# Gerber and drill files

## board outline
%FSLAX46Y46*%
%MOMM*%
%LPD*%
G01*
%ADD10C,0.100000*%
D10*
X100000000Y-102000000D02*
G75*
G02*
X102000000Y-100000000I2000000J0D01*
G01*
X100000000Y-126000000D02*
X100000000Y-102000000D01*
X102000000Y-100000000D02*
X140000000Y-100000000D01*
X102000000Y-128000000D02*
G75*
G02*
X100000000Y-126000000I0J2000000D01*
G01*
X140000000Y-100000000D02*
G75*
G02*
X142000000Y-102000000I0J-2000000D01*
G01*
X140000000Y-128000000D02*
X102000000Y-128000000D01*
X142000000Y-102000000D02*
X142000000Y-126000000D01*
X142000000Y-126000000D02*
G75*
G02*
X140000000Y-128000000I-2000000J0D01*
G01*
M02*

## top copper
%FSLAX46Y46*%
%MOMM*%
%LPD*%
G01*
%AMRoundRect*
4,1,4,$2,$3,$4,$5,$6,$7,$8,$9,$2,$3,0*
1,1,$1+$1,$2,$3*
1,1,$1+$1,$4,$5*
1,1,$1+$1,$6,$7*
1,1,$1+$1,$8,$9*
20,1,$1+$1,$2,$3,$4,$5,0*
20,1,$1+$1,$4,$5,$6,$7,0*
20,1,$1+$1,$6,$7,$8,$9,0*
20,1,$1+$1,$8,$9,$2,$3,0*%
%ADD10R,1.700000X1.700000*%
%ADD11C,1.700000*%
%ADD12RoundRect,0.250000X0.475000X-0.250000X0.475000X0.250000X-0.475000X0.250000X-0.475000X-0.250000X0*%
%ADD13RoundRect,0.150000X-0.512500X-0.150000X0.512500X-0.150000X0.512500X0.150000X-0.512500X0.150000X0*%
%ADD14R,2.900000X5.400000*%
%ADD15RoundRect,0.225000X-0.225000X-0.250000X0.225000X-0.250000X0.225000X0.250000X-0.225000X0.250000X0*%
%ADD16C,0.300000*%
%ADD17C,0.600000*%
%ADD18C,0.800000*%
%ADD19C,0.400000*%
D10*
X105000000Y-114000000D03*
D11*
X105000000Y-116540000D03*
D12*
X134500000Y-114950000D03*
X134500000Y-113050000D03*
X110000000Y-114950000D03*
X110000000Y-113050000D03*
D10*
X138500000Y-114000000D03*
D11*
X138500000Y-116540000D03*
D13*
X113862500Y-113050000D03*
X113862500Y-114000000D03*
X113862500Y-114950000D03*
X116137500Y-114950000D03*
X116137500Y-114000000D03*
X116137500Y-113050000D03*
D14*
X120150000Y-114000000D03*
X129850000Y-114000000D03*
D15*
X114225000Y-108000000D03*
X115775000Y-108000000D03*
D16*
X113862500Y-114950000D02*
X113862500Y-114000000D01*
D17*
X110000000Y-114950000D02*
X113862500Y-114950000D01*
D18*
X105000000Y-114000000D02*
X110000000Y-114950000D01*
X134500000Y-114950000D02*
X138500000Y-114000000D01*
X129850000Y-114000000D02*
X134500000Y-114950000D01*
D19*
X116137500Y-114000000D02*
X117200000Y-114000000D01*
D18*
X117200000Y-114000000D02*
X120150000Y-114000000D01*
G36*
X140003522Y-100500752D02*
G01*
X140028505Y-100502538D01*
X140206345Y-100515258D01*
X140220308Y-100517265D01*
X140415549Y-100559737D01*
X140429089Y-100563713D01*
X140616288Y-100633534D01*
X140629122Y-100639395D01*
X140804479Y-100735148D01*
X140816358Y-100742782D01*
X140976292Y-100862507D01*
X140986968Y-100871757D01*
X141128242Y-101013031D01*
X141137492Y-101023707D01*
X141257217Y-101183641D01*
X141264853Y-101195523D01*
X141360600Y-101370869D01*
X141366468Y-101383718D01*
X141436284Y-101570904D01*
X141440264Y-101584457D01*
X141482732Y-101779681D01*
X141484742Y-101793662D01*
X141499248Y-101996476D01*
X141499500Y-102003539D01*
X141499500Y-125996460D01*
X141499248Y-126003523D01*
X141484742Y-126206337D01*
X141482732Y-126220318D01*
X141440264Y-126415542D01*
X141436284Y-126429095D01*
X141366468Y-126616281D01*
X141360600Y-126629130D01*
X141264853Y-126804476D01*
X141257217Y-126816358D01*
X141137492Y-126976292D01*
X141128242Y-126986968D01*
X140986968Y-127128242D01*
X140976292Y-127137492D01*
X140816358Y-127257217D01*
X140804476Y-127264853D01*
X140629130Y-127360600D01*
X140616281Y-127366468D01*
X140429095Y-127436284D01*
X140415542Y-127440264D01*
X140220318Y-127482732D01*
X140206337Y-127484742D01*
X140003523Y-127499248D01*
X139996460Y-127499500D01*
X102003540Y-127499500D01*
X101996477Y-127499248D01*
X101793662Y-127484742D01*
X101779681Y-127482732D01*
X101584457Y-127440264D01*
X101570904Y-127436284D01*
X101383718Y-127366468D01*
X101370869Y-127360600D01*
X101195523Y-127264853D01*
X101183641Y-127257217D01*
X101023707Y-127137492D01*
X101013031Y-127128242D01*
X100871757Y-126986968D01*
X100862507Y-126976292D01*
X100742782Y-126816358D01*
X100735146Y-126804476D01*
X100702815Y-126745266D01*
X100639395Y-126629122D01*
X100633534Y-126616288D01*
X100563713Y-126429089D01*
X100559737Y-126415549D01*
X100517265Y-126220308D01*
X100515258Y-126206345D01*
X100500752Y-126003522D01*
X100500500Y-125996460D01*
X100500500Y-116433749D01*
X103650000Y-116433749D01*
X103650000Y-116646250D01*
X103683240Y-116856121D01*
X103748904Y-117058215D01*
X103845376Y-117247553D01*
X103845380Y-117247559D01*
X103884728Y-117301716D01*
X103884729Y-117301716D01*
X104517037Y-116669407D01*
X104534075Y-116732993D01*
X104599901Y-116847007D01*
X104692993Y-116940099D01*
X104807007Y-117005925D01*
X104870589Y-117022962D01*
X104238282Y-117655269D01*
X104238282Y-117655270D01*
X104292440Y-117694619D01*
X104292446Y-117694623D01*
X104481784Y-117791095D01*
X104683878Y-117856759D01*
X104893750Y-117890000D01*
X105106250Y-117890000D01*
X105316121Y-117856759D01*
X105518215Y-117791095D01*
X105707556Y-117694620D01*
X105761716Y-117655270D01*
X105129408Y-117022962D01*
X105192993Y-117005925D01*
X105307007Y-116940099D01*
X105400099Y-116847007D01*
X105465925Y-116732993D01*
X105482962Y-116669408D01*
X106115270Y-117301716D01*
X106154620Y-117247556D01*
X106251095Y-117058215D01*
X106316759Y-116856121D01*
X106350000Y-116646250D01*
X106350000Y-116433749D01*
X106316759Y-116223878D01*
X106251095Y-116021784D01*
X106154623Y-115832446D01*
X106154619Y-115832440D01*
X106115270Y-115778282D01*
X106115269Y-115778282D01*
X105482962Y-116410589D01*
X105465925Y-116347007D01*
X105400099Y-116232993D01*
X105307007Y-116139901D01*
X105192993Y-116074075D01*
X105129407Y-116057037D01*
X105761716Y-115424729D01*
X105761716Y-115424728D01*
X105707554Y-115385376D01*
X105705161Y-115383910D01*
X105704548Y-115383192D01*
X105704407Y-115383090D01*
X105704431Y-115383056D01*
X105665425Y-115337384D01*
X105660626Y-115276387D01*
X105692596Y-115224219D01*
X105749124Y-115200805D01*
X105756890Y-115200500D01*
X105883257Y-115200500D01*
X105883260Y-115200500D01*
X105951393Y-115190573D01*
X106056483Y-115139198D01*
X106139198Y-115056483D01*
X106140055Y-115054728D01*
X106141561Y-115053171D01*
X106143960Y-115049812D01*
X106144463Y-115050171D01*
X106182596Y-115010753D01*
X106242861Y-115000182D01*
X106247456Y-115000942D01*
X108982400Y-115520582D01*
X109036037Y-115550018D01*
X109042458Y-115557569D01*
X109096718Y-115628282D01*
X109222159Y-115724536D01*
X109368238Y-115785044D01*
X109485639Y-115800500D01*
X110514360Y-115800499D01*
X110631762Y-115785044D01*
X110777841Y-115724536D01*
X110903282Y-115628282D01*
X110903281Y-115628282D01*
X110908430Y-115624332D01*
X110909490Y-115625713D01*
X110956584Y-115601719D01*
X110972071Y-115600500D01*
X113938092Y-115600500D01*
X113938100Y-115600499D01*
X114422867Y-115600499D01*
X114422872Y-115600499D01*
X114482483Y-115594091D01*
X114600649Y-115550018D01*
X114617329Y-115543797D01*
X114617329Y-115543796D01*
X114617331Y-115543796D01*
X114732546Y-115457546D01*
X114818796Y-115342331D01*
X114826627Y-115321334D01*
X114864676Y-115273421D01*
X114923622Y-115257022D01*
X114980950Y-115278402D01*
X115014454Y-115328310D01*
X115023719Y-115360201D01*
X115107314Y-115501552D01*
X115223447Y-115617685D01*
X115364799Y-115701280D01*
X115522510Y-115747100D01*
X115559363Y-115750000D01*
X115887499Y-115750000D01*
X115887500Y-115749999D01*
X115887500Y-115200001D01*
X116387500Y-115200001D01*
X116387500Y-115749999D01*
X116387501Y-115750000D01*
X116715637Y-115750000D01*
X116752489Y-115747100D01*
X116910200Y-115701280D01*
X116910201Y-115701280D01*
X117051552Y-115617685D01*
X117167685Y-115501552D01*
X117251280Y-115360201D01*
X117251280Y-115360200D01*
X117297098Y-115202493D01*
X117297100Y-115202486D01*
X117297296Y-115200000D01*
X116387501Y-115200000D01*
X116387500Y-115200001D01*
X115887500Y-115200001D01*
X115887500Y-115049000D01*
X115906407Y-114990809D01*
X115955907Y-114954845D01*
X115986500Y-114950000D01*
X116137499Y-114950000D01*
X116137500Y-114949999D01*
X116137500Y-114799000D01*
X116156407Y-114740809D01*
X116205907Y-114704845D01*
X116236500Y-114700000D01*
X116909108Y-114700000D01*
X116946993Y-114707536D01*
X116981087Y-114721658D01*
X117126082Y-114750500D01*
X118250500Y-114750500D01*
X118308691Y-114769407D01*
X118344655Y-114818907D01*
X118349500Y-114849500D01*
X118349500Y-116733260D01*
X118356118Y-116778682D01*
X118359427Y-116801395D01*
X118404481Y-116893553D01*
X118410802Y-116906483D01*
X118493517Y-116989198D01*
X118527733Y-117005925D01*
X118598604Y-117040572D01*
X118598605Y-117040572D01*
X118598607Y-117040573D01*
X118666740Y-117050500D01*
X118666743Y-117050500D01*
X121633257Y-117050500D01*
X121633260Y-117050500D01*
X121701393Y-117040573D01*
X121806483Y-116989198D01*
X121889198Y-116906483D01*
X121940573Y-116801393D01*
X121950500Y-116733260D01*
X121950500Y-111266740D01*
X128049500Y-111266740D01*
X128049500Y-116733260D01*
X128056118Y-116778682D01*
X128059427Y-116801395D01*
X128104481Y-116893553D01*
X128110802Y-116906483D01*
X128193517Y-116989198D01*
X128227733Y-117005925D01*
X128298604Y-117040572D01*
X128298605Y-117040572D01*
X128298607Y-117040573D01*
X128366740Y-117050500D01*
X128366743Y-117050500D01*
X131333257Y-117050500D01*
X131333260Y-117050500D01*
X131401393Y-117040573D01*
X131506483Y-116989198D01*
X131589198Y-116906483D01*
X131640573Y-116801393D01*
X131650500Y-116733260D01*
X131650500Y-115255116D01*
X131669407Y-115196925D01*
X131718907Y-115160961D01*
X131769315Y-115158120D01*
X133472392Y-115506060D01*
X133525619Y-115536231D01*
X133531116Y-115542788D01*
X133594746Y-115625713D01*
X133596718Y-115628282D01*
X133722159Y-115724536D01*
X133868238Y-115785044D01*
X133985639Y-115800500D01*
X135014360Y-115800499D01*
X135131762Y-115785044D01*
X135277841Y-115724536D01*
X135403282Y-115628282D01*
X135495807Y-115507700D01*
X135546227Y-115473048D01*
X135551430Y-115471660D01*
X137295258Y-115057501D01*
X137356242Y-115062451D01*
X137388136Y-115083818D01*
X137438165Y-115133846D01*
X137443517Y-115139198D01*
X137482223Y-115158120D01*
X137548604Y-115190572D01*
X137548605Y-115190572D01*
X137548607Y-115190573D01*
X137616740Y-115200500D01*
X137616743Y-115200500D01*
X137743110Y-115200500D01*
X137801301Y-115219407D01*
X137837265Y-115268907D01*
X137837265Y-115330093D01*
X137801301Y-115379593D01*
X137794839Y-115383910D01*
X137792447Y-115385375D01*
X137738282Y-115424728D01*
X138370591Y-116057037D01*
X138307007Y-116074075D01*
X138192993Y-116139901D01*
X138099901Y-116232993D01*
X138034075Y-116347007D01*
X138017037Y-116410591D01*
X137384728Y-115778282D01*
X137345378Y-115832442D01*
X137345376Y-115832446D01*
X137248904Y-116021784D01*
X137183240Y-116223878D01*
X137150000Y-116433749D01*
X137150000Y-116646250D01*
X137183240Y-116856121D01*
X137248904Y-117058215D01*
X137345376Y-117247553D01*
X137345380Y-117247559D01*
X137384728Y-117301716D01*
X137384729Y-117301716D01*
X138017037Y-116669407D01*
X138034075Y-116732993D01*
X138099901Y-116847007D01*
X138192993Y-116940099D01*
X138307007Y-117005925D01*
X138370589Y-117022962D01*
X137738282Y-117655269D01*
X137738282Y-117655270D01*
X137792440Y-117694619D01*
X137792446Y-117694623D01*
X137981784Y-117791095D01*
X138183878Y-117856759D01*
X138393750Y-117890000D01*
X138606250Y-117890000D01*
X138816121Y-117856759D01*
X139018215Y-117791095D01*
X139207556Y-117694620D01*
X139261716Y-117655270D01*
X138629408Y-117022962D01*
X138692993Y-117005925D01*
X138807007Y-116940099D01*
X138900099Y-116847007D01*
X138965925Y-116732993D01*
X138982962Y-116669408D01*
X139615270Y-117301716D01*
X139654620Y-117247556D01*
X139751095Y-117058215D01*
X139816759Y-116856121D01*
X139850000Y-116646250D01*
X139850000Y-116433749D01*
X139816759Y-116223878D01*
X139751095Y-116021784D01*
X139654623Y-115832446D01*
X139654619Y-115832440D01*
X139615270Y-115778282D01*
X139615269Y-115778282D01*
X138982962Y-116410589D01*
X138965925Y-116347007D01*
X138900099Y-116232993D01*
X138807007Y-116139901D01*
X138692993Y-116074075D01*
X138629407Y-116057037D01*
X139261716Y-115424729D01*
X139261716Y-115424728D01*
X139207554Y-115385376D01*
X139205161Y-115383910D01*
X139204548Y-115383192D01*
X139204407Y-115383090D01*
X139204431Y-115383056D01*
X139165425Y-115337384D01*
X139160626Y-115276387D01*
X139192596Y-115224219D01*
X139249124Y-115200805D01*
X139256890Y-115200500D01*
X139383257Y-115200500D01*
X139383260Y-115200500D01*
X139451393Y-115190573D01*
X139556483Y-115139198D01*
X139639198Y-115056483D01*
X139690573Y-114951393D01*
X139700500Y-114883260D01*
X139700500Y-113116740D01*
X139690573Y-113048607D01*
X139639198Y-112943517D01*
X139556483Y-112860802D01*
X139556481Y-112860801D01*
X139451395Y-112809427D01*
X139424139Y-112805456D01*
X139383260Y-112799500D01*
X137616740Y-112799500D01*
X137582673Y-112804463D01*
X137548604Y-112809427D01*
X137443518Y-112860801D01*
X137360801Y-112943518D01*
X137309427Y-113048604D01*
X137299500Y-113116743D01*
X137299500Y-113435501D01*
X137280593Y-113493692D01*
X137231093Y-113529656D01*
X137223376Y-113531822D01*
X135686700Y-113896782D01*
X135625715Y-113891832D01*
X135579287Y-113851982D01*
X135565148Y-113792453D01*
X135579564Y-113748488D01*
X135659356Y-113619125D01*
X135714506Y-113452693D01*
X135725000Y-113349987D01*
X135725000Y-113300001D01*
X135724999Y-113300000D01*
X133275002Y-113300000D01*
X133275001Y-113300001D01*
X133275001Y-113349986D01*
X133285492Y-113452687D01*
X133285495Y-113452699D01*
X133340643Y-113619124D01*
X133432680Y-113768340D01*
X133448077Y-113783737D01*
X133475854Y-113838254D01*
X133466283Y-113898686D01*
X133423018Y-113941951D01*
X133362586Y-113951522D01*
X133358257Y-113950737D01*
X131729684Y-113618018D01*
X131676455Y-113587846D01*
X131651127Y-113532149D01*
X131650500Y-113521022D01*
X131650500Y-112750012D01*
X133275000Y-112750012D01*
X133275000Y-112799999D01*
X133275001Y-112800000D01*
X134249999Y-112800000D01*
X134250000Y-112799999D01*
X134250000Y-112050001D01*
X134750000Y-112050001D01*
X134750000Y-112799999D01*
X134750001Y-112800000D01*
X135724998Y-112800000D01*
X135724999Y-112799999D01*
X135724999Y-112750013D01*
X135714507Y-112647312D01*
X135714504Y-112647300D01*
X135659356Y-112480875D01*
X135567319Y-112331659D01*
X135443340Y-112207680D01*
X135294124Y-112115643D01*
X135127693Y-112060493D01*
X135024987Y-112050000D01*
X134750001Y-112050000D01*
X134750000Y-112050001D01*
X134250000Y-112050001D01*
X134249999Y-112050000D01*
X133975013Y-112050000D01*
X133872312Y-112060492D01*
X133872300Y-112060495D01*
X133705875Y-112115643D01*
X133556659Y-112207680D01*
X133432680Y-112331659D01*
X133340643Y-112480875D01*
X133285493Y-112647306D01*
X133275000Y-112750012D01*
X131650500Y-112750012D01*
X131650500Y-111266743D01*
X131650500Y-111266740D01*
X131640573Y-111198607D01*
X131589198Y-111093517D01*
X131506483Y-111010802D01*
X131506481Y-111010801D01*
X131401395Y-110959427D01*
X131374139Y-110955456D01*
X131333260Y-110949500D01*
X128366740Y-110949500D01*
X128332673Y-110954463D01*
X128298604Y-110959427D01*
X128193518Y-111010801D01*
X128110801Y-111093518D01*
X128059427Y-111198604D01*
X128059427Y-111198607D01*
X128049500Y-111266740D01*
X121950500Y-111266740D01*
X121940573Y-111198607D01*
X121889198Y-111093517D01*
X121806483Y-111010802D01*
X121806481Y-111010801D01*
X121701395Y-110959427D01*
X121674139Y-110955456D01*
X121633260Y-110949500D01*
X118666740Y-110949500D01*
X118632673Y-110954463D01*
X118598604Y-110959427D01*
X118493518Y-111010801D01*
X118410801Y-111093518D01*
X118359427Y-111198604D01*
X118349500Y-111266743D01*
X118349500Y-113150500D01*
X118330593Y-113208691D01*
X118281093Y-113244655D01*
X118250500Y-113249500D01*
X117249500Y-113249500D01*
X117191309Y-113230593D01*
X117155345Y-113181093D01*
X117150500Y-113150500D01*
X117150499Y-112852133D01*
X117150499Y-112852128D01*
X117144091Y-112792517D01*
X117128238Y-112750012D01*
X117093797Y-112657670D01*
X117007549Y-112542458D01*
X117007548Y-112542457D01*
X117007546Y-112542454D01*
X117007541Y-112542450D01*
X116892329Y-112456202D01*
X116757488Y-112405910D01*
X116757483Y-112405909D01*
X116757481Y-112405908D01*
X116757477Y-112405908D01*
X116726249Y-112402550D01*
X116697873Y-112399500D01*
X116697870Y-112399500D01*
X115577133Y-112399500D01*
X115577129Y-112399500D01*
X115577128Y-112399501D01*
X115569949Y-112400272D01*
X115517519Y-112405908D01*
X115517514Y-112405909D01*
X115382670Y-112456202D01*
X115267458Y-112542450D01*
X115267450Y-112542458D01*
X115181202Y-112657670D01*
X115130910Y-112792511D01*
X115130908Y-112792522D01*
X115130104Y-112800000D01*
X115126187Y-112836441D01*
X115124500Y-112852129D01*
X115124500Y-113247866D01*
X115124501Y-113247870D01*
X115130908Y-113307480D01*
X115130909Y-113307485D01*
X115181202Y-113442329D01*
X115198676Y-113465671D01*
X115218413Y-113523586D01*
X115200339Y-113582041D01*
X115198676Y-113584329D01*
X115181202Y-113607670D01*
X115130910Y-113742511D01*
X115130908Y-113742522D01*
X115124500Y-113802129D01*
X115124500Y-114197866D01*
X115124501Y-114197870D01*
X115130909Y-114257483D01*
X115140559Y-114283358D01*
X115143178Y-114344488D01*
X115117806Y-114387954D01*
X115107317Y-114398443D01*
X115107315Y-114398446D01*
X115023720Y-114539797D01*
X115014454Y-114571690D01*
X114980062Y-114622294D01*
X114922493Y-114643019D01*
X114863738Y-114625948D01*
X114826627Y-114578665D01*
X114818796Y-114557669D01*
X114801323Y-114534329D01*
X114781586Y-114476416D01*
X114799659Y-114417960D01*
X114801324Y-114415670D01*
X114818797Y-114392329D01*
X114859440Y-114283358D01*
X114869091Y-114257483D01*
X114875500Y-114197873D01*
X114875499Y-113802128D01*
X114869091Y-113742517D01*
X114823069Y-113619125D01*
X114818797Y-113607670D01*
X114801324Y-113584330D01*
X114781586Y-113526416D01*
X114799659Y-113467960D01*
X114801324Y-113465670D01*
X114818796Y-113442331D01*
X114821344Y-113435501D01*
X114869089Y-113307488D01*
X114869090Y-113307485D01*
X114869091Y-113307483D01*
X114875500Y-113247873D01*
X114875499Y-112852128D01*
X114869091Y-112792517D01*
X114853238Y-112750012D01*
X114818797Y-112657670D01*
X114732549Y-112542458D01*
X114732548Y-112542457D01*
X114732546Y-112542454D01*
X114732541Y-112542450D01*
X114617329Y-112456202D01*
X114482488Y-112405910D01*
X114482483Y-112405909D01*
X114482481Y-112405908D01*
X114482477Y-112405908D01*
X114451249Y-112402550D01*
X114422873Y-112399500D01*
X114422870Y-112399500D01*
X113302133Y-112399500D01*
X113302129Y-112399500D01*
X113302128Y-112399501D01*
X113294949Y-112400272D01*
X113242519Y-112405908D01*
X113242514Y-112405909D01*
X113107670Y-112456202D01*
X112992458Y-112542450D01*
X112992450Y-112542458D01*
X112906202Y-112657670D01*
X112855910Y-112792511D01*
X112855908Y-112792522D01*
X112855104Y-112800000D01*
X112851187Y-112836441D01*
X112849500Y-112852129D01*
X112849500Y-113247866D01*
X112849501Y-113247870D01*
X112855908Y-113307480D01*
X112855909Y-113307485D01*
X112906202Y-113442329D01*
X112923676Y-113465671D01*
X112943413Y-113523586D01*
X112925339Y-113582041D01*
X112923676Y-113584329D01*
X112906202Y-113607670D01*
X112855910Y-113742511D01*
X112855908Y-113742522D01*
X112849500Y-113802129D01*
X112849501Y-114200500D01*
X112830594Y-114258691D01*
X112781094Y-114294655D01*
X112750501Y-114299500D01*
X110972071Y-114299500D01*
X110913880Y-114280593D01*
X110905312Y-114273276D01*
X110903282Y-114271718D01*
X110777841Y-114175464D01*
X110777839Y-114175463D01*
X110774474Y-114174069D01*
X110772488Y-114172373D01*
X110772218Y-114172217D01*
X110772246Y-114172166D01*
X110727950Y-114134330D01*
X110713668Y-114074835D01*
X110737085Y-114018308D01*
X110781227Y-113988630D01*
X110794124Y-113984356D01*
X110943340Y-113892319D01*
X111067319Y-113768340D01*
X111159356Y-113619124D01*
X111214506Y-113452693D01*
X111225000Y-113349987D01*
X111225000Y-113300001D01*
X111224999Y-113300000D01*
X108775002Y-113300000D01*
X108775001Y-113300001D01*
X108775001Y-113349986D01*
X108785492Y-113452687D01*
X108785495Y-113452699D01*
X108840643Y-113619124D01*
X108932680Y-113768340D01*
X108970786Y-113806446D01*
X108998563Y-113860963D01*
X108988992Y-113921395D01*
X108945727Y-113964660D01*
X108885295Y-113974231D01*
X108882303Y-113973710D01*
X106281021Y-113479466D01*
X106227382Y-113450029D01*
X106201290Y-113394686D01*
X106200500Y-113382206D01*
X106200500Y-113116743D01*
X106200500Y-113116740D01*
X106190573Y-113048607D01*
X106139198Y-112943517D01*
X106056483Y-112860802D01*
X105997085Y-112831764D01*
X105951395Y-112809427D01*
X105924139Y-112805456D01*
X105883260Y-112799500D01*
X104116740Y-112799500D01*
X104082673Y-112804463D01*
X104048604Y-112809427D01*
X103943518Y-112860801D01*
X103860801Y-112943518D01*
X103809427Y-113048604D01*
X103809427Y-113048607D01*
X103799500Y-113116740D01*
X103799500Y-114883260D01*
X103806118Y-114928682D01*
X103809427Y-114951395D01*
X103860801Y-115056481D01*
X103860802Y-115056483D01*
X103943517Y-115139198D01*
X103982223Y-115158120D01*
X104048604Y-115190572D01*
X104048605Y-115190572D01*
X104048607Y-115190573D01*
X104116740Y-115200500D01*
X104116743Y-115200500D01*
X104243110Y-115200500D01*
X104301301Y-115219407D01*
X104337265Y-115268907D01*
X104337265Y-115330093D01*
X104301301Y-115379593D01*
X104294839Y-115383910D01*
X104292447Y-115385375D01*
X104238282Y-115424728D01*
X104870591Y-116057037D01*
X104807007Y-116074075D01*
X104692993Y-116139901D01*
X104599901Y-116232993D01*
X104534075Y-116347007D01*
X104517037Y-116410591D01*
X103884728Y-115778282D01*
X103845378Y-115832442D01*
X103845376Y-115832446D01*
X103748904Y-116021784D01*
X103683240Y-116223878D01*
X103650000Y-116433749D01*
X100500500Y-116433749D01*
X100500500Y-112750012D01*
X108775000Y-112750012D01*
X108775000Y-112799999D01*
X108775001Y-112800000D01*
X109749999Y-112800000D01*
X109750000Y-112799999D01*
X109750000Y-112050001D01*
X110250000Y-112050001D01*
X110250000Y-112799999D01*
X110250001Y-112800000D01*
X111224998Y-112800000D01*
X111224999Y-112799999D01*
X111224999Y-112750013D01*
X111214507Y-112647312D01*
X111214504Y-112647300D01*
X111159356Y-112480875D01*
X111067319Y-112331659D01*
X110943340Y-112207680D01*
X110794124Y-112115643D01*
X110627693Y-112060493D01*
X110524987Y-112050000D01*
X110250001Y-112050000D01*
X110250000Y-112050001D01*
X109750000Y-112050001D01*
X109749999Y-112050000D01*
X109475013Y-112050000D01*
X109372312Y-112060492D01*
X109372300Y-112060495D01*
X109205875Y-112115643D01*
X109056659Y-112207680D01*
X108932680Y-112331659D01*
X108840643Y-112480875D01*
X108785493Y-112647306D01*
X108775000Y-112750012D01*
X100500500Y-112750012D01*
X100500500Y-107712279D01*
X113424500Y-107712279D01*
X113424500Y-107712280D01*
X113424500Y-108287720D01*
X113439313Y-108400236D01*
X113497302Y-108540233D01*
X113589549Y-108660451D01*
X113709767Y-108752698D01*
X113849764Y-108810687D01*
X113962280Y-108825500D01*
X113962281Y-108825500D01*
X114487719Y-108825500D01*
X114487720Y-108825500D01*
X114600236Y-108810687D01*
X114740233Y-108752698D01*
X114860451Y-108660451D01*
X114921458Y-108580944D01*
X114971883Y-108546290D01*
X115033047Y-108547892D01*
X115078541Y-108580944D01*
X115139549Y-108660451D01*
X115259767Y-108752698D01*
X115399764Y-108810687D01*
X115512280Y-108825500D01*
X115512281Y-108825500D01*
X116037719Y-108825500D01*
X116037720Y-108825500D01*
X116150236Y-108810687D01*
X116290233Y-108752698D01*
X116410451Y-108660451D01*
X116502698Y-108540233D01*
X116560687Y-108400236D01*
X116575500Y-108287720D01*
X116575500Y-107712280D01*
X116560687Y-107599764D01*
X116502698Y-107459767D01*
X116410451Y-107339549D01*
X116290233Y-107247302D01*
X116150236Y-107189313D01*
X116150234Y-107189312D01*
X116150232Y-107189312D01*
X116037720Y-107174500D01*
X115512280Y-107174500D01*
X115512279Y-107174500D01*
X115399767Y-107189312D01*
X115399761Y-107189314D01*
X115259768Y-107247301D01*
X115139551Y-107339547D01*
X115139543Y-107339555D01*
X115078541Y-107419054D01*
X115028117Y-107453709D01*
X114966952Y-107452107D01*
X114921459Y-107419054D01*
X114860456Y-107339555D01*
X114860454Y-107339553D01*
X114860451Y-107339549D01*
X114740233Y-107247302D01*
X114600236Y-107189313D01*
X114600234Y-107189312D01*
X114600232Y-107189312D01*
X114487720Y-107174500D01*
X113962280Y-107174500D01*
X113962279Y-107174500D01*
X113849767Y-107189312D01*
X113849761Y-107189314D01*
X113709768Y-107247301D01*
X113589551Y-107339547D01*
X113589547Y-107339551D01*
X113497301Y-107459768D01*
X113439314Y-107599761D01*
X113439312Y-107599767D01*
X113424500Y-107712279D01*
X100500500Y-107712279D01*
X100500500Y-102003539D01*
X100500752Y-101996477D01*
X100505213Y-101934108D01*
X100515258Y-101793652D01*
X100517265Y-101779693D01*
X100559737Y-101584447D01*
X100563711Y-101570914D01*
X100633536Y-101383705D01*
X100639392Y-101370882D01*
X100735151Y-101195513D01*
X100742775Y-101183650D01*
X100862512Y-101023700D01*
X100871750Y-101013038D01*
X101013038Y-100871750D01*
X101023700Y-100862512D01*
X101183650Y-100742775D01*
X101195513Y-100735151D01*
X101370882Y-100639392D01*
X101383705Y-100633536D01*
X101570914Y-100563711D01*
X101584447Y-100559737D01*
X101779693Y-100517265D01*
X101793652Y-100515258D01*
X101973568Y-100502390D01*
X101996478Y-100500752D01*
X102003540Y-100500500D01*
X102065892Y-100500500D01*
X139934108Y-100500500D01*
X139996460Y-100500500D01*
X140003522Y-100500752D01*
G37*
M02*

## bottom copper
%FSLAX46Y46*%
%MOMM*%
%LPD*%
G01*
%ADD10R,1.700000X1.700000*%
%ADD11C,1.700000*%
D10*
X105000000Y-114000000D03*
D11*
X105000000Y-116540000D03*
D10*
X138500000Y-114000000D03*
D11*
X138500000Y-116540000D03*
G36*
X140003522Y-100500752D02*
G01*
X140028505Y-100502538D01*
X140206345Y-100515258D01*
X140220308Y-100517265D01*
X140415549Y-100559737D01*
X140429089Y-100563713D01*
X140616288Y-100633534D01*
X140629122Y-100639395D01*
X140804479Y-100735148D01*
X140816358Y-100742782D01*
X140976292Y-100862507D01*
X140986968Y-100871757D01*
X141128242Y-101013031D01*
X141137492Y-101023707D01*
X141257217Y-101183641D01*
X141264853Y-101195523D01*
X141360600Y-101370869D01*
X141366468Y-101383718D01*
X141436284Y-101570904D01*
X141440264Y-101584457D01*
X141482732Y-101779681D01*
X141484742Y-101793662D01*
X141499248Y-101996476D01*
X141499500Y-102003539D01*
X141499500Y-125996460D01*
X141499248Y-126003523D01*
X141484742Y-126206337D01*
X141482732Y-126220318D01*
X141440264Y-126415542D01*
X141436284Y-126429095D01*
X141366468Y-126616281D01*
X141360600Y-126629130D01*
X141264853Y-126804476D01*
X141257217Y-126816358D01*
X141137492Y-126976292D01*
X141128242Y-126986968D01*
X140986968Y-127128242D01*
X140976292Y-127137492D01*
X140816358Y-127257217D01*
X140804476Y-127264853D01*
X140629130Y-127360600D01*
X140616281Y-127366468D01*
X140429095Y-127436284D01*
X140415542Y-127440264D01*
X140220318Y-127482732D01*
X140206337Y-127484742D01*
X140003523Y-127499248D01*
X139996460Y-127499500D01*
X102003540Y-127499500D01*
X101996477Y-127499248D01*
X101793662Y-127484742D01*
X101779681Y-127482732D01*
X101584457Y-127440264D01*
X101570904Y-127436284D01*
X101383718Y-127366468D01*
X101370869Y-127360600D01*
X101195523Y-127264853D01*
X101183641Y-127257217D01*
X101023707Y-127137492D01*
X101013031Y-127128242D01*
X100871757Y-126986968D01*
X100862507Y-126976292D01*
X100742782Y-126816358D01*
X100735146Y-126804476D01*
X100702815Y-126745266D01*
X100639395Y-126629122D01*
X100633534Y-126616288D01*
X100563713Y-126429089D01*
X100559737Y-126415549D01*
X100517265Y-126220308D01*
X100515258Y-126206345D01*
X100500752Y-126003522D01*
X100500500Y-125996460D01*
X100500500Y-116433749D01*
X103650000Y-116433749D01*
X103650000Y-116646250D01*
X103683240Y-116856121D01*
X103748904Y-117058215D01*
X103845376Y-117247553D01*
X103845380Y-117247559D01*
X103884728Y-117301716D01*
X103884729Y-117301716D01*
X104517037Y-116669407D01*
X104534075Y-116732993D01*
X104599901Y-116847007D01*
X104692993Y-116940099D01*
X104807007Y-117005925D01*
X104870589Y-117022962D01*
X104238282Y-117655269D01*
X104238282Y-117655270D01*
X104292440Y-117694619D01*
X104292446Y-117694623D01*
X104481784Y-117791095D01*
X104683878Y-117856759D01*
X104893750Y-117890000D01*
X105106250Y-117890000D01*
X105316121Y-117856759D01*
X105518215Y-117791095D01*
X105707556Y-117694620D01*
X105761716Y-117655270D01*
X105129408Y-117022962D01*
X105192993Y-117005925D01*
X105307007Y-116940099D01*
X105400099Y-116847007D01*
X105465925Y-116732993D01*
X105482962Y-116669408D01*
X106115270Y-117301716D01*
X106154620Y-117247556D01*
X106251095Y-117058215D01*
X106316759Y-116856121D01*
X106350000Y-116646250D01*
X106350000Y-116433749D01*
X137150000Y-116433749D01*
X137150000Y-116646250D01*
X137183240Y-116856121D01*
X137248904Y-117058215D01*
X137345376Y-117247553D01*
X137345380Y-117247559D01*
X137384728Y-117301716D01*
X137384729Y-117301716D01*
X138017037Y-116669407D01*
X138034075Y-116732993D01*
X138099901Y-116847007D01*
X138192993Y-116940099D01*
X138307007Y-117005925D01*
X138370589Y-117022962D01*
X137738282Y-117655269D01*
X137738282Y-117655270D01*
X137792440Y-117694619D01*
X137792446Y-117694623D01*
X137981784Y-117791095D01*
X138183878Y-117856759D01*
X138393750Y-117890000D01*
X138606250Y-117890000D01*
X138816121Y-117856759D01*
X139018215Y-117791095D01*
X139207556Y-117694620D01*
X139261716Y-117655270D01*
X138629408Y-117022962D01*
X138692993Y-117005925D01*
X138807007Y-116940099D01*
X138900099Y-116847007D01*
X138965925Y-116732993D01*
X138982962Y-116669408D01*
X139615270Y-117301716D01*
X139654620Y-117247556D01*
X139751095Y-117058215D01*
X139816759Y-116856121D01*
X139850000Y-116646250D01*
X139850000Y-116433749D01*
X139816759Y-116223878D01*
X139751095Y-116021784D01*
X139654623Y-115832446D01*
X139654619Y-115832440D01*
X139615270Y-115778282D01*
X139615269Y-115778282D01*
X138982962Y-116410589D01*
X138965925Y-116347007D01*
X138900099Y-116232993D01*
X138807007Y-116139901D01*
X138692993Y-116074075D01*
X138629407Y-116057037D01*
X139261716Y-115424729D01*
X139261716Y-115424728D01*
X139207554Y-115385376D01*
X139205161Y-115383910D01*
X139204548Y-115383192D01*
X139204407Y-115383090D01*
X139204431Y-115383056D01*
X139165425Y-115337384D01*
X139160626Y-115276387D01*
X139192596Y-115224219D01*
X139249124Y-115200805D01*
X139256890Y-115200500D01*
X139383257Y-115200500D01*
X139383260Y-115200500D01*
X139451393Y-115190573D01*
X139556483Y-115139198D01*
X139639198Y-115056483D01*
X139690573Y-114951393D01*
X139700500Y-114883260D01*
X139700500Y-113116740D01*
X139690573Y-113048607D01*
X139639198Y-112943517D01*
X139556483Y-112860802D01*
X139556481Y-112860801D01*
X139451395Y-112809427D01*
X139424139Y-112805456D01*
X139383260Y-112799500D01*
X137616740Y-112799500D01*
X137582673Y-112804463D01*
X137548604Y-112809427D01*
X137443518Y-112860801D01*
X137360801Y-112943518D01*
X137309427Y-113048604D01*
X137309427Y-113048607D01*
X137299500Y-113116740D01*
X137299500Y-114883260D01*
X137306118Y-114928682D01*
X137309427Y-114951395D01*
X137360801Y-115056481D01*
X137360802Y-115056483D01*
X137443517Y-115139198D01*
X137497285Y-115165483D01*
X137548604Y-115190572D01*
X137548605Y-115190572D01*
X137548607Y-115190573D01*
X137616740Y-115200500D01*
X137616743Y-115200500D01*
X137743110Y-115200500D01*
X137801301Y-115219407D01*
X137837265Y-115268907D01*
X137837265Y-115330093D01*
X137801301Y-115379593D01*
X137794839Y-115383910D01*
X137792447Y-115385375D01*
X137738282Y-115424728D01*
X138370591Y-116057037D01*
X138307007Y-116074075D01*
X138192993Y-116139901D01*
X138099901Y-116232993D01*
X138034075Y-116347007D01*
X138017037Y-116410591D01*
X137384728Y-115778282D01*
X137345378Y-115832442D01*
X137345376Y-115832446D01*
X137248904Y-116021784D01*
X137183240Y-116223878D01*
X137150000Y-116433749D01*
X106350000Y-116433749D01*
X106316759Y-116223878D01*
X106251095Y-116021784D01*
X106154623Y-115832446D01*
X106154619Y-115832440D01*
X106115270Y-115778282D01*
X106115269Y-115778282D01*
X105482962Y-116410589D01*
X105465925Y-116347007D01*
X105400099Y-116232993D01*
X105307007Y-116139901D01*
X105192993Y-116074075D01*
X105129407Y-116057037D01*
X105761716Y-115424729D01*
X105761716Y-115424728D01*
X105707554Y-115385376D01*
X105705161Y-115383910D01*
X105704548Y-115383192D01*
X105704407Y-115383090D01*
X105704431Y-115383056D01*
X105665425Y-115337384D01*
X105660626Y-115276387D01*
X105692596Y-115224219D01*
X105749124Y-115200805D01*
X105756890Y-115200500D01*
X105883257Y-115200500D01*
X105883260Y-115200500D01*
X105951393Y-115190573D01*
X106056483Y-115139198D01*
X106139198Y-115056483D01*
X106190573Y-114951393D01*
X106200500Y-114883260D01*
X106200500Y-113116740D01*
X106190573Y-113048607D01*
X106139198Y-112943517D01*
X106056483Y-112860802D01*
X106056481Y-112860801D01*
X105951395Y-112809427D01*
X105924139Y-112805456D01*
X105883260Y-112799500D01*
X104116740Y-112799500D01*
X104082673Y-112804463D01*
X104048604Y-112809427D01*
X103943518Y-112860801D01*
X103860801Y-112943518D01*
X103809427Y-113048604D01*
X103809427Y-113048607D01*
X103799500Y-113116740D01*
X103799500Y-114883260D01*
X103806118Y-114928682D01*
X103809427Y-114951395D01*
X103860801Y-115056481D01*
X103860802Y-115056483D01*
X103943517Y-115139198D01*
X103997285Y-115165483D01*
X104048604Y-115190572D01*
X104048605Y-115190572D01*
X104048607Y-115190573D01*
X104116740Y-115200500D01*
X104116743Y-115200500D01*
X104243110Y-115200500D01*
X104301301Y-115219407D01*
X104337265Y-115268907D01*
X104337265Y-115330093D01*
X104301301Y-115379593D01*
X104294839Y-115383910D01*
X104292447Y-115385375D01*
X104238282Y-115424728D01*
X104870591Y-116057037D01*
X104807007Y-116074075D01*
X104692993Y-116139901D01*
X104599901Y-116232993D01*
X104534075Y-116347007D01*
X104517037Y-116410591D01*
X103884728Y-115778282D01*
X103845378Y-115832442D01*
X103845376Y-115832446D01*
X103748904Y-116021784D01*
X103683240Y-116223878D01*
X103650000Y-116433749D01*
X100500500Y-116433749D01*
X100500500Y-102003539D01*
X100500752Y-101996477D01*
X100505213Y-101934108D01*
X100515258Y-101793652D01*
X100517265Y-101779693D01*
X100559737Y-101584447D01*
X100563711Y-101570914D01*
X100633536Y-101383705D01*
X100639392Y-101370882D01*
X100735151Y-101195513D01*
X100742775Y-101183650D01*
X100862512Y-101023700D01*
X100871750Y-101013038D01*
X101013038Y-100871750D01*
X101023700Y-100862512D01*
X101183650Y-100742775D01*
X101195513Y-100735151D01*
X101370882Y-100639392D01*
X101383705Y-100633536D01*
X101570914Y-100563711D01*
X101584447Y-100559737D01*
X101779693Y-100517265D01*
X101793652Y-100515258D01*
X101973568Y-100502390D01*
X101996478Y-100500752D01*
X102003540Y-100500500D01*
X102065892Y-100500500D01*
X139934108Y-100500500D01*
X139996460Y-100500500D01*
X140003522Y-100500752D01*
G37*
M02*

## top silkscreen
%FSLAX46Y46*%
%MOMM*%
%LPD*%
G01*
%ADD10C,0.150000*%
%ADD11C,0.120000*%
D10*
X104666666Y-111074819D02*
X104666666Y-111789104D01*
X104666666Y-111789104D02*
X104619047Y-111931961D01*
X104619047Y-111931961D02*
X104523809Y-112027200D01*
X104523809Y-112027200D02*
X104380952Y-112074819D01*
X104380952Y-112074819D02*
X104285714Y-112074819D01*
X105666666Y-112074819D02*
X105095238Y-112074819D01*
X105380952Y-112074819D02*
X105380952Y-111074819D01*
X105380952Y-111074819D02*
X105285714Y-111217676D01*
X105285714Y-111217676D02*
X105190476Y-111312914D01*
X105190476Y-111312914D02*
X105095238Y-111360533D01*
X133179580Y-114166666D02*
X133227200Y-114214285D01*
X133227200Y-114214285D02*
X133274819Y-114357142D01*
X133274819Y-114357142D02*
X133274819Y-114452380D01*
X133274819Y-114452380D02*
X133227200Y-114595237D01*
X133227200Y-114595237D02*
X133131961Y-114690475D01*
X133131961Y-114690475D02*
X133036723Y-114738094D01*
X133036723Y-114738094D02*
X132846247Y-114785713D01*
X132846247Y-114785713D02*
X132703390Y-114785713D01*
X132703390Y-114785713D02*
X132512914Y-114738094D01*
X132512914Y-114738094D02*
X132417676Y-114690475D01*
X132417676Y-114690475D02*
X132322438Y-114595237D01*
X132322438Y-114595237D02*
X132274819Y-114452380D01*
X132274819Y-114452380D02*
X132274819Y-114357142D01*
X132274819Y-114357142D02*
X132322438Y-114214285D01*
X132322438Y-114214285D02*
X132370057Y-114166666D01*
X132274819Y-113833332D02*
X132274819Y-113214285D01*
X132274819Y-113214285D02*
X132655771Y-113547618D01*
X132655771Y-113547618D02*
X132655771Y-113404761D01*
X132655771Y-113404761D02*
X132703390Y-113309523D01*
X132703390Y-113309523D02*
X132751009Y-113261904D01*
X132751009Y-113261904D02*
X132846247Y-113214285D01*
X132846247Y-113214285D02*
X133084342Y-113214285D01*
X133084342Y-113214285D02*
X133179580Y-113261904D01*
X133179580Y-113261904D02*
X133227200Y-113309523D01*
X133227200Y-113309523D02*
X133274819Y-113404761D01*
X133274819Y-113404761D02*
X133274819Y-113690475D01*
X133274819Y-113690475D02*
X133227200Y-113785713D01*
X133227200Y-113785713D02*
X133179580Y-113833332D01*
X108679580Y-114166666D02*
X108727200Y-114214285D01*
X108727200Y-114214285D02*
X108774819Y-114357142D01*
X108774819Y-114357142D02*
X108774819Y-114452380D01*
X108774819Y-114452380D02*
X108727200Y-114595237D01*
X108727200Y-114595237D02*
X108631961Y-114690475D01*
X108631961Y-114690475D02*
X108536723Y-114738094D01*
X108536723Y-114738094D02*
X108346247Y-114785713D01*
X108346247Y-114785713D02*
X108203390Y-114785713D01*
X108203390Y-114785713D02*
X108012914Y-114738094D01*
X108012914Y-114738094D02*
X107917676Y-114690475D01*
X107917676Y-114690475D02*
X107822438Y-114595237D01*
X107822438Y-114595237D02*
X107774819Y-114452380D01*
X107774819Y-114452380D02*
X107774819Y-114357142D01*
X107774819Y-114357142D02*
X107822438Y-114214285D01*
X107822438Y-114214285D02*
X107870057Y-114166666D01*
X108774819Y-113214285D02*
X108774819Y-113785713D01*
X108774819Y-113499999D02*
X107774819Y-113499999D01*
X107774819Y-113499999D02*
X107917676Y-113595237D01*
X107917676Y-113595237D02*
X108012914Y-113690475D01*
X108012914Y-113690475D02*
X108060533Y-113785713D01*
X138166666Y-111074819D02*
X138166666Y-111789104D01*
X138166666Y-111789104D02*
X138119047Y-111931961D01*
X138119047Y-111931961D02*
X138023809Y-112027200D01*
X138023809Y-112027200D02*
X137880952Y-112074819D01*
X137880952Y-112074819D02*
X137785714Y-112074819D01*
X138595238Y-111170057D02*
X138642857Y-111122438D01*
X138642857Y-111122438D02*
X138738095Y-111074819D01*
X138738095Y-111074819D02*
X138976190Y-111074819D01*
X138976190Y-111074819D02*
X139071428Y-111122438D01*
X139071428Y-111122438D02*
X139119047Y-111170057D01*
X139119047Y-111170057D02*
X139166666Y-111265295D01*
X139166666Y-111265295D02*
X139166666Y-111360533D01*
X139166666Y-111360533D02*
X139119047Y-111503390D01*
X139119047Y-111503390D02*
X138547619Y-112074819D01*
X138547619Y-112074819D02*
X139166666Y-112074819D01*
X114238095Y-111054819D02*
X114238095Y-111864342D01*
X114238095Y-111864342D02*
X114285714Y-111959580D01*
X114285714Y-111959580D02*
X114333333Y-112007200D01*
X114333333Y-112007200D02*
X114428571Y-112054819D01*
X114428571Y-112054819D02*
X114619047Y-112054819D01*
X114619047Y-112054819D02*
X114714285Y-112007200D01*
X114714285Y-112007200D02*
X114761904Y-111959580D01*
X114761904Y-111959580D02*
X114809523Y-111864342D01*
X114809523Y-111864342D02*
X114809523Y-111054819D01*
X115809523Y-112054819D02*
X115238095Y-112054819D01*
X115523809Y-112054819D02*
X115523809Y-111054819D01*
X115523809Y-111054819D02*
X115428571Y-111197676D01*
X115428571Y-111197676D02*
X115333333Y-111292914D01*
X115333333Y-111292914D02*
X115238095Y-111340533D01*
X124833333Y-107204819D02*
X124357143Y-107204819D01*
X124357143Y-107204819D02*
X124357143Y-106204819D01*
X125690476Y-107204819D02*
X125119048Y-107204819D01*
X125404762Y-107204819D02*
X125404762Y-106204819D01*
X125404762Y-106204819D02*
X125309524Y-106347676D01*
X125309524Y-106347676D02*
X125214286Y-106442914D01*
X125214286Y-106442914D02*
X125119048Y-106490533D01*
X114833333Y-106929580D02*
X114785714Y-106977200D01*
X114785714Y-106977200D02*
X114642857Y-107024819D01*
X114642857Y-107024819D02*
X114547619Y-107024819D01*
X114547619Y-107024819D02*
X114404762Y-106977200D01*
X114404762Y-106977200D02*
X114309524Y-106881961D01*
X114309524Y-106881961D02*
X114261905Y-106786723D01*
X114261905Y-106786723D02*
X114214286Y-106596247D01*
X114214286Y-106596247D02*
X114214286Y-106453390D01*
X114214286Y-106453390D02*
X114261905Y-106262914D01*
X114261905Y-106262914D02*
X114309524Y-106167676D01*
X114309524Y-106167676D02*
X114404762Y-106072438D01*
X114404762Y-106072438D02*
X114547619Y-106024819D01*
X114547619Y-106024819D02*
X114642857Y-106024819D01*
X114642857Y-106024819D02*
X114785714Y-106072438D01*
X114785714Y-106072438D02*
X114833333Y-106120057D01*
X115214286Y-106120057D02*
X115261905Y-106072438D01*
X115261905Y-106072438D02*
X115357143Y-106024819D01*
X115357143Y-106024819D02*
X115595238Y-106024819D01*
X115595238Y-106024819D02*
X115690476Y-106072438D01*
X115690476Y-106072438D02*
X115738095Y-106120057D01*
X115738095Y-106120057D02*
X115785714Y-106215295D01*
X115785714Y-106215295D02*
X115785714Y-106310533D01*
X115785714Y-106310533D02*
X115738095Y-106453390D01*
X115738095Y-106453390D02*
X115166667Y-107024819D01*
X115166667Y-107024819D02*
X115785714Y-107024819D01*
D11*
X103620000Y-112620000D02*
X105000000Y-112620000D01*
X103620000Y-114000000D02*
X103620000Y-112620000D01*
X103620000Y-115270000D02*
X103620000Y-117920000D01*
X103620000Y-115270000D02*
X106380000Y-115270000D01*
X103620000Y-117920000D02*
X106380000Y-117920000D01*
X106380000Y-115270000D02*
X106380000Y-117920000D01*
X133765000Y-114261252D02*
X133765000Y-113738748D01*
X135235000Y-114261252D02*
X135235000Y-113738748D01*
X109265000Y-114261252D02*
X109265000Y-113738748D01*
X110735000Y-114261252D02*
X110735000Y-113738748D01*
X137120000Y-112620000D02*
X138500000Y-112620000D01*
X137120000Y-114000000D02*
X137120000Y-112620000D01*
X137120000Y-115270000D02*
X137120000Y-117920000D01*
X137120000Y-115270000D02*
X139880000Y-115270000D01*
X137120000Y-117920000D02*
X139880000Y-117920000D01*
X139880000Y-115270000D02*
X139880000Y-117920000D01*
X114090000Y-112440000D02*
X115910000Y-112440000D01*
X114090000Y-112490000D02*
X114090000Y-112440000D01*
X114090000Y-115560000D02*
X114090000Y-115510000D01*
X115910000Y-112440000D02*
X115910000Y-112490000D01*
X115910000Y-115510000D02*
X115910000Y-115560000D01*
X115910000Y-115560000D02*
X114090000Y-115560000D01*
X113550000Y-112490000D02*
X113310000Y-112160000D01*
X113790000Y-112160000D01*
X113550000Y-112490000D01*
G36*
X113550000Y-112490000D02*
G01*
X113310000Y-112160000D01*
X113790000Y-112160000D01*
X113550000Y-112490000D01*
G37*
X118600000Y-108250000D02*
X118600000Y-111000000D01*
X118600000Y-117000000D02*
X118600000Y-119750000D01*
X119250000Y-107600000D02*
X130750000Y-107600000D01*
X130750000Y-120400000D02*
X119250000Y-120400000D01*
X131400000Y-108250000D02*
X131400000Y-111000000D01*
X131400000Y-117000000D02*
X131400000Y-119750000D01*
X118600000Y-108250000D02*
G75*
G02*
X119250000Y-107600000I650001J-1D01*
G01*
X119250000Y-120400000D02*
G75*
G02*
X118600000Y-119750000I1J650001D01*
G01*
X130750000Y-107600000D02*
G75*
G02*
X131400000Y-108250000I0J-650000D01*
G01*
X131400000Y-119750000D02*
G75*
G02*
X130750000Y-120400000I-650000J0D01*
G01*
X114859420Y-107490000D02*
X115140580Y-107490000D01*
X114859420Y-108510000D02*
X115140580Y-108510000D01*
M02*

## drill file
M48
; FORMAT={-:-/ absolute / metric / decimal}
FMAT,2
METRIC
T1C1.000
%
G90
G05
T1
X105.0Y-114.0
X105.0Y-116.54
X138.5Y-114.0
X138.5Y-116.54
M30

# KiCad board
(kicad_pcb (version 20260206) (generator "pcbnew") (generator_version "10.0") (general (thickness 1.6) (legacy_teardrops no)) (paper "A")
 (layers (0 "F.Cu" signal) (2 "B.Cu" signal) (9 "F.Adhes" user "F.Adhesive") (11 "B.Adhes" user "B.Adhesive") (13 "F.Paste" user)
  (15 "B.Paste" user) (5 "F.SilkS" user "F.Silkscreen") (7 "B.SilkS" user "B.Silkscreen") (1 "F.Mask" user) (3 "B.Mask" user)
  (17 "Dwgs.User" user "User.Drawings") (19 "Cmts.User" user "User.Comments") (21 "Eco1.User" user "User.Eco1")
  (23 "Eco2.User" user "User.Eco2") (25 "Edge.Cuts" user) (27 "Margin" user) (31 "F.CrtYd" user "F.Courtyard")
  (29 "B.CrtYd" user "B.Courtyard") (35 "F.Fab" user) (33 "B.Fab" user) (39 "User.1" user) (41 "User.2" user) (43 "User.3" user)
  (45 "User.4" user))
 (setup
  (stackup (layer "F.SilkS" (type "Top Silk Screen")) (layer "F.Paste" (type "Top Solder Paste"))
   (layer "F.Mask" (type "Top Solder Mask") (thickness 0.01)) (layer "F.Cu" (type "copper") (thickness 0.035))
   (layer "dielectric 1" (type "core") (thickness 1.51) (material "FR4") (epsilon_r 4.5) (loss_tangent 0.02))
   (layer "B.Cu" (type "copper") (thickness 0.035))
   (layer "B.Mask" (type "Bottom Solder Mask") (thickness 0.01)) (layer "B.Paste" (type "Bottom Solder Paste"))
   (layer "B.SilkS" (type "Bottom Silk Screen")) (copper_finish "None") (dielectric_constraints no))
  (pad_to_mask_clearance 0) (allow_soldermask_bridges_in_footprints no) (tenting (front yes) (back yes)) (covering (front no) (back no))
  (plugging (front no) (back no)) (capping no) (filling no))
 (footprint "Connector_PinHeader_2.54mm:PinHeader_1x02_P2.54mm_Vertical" (layer "F.Cu") (at 105 114)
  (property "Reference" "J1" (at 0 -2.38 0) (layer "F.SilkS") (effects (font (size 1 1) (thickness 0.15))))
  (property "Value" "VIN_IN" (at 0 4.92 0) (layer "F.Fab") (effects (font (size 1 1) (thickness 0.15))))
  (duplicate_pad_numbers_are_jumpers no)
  (fp_line (start -1.38 -1.38) (end 0 -1.38) (stroke (width 0.12) (type solid)) (layer "F.SilkS"))
  (fp_line (start -1.38 0) (end -1.38 -1.38) (stroke (width 0.12) (type solid)) (layer "F.SilkS"))
  (fp_line (start -1.38 1.27) (end -1.38 3.92) (stroke (width 0.12) (type solid)) (layer "F.SilkS"))
  (fp_line (start -1.38 1.27) (end 1.38 1.27) (stroke (width 0.12) (type solid)) (layer "F.SilkS"))
  (fp_line (start -1.38 3.92) (end 1.38 3.92) (stroke (width 0.12) (type solid)) (layer "F.SilkS"))
  (fp_line (start 1.38 1.27) (end 1.38 3.92) (stroke (width 0.12) (type solid)) (layer "F.SilkS"))
  (pad "1" thru_hole rect (at 0 0) (size 1.7 1.7) (drill 1) (layers "*.Cu" "*.Mask") (remove_unused_layers no) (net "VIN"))
  (pad "2" thru_hole circle (at 0 2.54) (size 1.7 1.7) (drill 1) (layers "*.Cu" "*.Mask") (remove_unused_layers no) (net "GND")))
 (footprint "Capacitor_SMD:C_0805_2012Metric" (layer "F.Cu") (at 134.5 114 90)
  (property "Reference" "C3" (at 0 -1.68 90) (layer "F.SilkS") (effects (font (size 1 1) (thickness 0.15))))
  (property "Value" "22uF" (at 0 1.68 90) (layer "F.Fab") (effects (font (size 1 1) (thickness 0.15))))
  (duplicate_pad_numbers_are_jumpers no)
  (fp_line (start -0.261252 -0.735) (end 0.261252 -0.735) (stroke (width 0.12) (type solid)) (layer "F.SilkS"))
  (fp_line (start -0.261252 0.735) (end 0.261252 0.735) (stroke (width 0.12) (type solid)) (layer "F.SilkS"))
  (pad "1" smd roundrect (at -0.95 0 90) (size 1 1.45) (layers "F.Cu" "F.Mask" "F.Paste") (roundrect_rratio 0.25) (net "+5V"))
  (pad "2" smd roundrect (at 0.95 0 90) (size 1 1.45) (layers "F.Cu" "F.Mask" "F.Paste") (roundrect_rratio 0.25) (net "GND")))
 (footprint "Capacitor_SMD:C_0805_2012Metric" (layer "F.Cu") (at 110 114 90)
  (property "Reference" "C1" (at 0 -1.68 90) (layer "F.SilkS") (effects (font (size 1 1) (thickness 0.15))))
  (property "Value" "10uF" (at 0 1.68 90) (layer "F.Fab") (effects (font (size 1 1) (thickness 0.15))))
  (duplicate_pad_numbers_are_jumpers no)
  (fp_line (start -0.261252 -0.735) (end 0.261252 -0.735) (stroke (width 0.12) (type solid)) (layer "F.SilkS"))
  (fp_line (start -0.261252 0.735) (end 0.261252 0.735) (stroke (width 0.12) (type solid)) (layer "F.SilkS"))
  (pad "1" smd roundrect (at -0.95 0 90) (size 1 1.45) (layers "F.Cu" "F.Mask" "F.Paste") (roundrect_rratio 0.25) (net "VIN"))
  (pad "2" smd roundrect (at 0.95 0 90) (size 1 1.45) (layers "F.Cu" "F.Mask" "F.Paste") (roundrect_rratio 0.25) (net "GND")))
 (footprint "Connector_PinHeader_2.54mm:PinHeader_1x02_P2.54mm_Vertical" (layer "F.Cu") (at 138.5 114)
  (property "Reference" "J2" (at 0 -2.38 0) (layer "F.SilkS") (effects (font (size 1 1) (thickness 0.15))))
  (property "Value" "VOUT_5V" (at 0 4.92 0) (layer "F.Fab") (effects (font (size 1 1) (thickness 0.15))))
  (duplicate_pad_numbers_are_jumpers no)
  (fp_line (start -1.38 -1.38) (end 0 -1.38) (stroke (width 0.12) (type solid)) (layer "F.SilkS"))
  (fp_line (start -1.38 0) (end -1.38 -1.38) (stroke (width 0.12) (type solid)) (layer "F.SilkS"))
  (fp_line (start -1.38 1.27) (end -1.38 3.92) (stroke (width 0.12) (type solid)) (layer "F.SilkS"))
  (fp_line (start -1.38 1.27) (end 1.38 1.27) (stroke (width 0.12) (type solid)) (layer "F.SilkS"))
  (fp_line (start -1.38 3.92) (end 1.38 3.92) (stroke (width 0.12) (type solid)) (layer "F.SilkS"))
  (fp_line (start 1.38 1.27) (end 1.38 3.92) (stroke (width 0.12) (type solid)) (layer "F.SilkS"))
  (pad "1" thru_hole rect (at 0 0) (size 1.7 1.7) (drill 1) (layers "*.Cu" "*.Mask") (remove_unused_layers no) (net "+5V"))
  (pad "2" thru_hole circle (at 0 2.54) (size 1.7 1.7) (drill 1) (layers "*.Cu" "*.Mask") (remove_unused_layers no) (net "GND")))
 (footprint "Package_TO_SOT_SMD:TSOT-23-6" (layer "F.Cu") (at 115 114)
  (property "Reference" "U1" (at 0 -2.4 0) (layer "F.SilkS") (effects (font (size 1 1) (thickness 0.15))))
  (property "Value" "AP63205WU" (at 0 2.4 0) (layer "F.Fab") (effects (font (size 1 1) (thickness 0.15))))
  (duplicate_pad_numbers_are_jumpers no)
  (fp_line (start -0.91 -1.56) (end 0.91 -1.56) (stroke (width 0.12) (type solid)) (layer "F.SilkS"))
  (fp_line (start -0.91 -1.51) (end -0.91 -1.56) (stroke (width 0.12) (type solid)) (layer "F.SilkS"))
  (fp_line (start -0.91 1.56) (end -0.91 1.51) (stroke (width 0.12) (type solid)) (layer "F.SilkS"))
  (fp_line (start 0.91 -1.56) (end 0.91 -1.51) (stroke (width 0.12) (type solid)) (layer "F.SilkS"))
  (fp_line (start 0.91 1.51) (end 0.91 1.56) (stroke (width 0.12) (type solid)) (layer "F.SilkS"))
  (fp_line (start 0.91 1.56) (end -0.91 1.56) (stroke (width 0.12) (type solid)) (layer "F.SilkS"))
  (fp_poly (pts (xy -1.45 -1.51) (xy -1.69 -1.84) (xy -1.21 -1.84)) (stroke (width 0.12) (type solid)) (fill yes) (layer "F.SilkS"))
  (pad "1" smd roundrect (at -1.1375 -0.95) (size 1.325 0.6) (layers "F.Cu" "F.Mask" "F.Paste") (roundrect_rratio 0.25) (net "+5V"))
  (pad "2" smd roundrect (at -1.1375 0) (size 1.325 0.6) (layers "F.Cu" "F.Mask" "F.Paste") (roundrect_rratio 0.25) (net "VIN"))
  (pad "3" smd roundrect (at -1.1375 0.95) (size 1.325 0.6) (layers "F.Cu" "F.Mask" "F.Paste") (roundrect_rratio 0.25) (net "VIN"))
  (pad "4" smd roundrect (at 1.1375 0.95) (size 1.325 0.6) (layers "F.Cu" "F.Mask" "F.Paste") (roundrect_rratio 0.25) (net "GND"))
  (pad "5" smd roundrect (at 1.1375 0) (size 1.325 0.6) (layers "F.Cu" "F.Mask" "F.Paste") (roundrect_rratio 0.25) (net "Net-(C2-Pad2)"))
  (pad "6" smd roundrect (at 1.1375 -0.95) (size 1.325 0.6) (layers "F.Cu" "F.Mask" "F.Paste") (roundrect_rratio 0.25) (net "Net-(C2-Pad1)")))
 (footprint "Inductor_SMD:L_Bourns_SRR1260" (layer "F.Cu") (at 125 114)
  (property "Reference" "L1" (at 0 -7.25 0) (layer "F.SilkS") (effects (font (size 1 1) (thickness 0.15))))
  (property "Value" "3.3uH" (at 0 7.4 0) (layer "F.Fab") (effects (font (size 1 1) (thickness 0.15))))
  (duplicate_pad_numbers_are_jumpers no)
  (fp_line (start -6.4 -5.75) (end -6.4 -3) (stroke (width 0.12) (type solid)) (layer "F.SilkS"))
  (fp_line (start -6.4 3) (end -6.4 5.75) (stroke (width 0.12) (type solid)) (layer "F.SilkS"))
  (fp_line (start -5.75 -6.4) (end 5.75 -6.4) (stroke (width 0.12) (type solid)) (layer "F.SilkS"))
  (fp_line (start 5.75 6.4) (end -5.75 6.4) (stroke (width 0.12) (type solid)) (layer "F.SilkS"))
  (fp_line (start 6.4 -5.75) (end 6.4 -3) (stroke (width 0.12) (type solid)) (layer "F.SilkS"))
  (fp_line (start 6.4 3) (end 6.4 5.75) (stroke (width 0.12) (type solid)) (layer "F.SilkS"))
  (fp_arc (start -6.4 -5.75) (mid -6.209619 -6.209619) (end -5.75 -6.4) (stroke (width 0.12) (type solid)) (layer "F.SilkS"))
  (fp_arc (start -5.75 6.4) (mid -6.209619 6.209619) (end -6.4 5.75) (stroke (width 0.12) (type solid)) (layer "F.SilkS"))
  (fp_arc (start 5.75 -6.4) (mid 6.209619 -6.209619) (end 6.4 -5.75) (stroke (width 0.12) (type solid)) (layer "F.SilkS"))
  (fp_arc (start 6.4 5.75) (mid 6.209619 6.209619) (end 5.75 6.4) (stroke (width 0.12) (type solid)) (layer "F.SilkS"))
  (pad "1" smd rect (at -4.85 0) (size 2.9 5.4) (layers "F.Cu" "F.Mask" "F.Paste") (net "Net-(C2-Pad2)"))
  (pad "2" smd rect (at 4.85 0) (size 2.9 5.4) (layers "F.Cu" "F.Mask" "F.Paste") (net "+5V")))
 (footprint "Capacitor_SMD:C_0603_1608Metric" (layer "F.Cu") (at 115 108)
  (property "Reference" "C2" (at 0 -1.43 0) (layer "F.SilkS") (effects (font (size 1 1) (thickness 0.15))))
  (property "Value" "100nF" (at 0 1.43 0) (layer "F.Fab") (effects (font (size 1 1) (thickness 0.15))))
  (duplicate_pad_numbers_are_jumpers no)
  (fp_line (start -0.14058 -0.51) (end 0.14058 -0.51) (stroke (width 0.12) (type solid)) (layer "F.SilkS"))
  (fp_line (start -0.14058 0.51) (end 0.14058 0.51) (stroke (width 0.12) (type solid)) (layer "F.SilkS"))
  (pad "1" smd roundrect (at -0.775 0) (size 0.9 0.95) (layers "F.Cu" "F.Mask" "F.Paste") (roundrect_rratio 0.25) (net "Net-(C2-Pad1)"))
  (pad "2" smd roundrect (at 0.775 0) (size 0.9 0.95) (layers "F.Cu" "F.Mask" "F.Paste") (roundrect_rratio 0.25) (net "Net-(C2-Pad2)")))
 (gr_arc (start 100 102) (mid 100.585786 100.585786) (end 102 100) (stroke (width 0.1) (type default)) (layer "Edge.Cuts"))
 (gr_line (start 100 126) (end 100 102) (stroke (width 0.1) (type default)) (layer "Edge.Cuts"))
 (gr_line (start 102 100) (end 140 100) (stroke (width 0.1) (type default)) (layer "Edge.Cuts"))
 (gr_arc (start 102 128) (mid 100.585786 127.414214) (end 100 126) (stroke (width 0.1) (type default)) (layer "Edge.Cuts"))
 (gr_arc (start 140 100) (mid 141.414214 100.585786) (end 142 102) (stroke (width 0.1) (type default)) (layer "Edge.Cuts"))
 (gr_line (start 140 128) (end 102 128) (stroke (width 0.1) (type default)) (layer "Edge.Cuts"))
 (gr_line (start 142 102) (end 142 126) (stroke (width 0.1) (type default)) (layer "Edge.Cuts"))
 (gr_arc (start 142 126) (mid 141.414214 127.414214) (end 140 128) (stroke (width 0.1) (type default)) (layer "Edge.Cuts"))
 (segment (start 113.8625 114.95) (end 113.8625 114) (width 0.3) (layer "F.Cu") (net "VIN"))
 (segment (start 110 114.95) (end 113.8625 114.95) (width 0.6) (layer "F.Cu") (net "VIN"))
 (segment (start 105 114) (end 110 114.95) (width 0.8) (layer "F.Cu") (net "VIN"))
 (segment (start 134.5 114.95) (end 138.5 114) (width 0.8) (layer "F.Cu") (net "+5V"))
 (segment (start 129.85 114) (end 134.5 114.95) (width 0.8) (layer "F.Cu") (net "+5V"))
 (segment (start 116.1375 114) (end 117.2 114) (width 0.4) (layer "F.Cu") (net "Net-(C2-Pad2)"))
 (segment (start 117.2 114) (end 120.15 114) (width 0.8) (layer "F.Cu") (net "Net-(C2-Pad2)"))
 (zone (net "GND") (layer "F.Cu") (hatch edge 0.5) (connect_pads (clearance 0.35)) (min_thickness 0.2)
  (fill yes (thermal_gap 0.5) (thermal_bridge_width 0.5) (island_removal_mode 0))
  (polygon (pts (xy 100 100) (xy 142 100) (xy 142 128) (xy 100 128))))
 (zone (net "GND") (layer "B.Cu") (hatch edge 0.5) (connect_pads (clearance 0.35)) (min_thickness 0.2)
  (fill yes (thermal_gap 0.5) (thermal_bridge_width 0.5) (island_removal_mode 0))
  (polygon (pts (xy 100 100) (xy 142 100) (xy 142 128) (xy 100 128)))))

